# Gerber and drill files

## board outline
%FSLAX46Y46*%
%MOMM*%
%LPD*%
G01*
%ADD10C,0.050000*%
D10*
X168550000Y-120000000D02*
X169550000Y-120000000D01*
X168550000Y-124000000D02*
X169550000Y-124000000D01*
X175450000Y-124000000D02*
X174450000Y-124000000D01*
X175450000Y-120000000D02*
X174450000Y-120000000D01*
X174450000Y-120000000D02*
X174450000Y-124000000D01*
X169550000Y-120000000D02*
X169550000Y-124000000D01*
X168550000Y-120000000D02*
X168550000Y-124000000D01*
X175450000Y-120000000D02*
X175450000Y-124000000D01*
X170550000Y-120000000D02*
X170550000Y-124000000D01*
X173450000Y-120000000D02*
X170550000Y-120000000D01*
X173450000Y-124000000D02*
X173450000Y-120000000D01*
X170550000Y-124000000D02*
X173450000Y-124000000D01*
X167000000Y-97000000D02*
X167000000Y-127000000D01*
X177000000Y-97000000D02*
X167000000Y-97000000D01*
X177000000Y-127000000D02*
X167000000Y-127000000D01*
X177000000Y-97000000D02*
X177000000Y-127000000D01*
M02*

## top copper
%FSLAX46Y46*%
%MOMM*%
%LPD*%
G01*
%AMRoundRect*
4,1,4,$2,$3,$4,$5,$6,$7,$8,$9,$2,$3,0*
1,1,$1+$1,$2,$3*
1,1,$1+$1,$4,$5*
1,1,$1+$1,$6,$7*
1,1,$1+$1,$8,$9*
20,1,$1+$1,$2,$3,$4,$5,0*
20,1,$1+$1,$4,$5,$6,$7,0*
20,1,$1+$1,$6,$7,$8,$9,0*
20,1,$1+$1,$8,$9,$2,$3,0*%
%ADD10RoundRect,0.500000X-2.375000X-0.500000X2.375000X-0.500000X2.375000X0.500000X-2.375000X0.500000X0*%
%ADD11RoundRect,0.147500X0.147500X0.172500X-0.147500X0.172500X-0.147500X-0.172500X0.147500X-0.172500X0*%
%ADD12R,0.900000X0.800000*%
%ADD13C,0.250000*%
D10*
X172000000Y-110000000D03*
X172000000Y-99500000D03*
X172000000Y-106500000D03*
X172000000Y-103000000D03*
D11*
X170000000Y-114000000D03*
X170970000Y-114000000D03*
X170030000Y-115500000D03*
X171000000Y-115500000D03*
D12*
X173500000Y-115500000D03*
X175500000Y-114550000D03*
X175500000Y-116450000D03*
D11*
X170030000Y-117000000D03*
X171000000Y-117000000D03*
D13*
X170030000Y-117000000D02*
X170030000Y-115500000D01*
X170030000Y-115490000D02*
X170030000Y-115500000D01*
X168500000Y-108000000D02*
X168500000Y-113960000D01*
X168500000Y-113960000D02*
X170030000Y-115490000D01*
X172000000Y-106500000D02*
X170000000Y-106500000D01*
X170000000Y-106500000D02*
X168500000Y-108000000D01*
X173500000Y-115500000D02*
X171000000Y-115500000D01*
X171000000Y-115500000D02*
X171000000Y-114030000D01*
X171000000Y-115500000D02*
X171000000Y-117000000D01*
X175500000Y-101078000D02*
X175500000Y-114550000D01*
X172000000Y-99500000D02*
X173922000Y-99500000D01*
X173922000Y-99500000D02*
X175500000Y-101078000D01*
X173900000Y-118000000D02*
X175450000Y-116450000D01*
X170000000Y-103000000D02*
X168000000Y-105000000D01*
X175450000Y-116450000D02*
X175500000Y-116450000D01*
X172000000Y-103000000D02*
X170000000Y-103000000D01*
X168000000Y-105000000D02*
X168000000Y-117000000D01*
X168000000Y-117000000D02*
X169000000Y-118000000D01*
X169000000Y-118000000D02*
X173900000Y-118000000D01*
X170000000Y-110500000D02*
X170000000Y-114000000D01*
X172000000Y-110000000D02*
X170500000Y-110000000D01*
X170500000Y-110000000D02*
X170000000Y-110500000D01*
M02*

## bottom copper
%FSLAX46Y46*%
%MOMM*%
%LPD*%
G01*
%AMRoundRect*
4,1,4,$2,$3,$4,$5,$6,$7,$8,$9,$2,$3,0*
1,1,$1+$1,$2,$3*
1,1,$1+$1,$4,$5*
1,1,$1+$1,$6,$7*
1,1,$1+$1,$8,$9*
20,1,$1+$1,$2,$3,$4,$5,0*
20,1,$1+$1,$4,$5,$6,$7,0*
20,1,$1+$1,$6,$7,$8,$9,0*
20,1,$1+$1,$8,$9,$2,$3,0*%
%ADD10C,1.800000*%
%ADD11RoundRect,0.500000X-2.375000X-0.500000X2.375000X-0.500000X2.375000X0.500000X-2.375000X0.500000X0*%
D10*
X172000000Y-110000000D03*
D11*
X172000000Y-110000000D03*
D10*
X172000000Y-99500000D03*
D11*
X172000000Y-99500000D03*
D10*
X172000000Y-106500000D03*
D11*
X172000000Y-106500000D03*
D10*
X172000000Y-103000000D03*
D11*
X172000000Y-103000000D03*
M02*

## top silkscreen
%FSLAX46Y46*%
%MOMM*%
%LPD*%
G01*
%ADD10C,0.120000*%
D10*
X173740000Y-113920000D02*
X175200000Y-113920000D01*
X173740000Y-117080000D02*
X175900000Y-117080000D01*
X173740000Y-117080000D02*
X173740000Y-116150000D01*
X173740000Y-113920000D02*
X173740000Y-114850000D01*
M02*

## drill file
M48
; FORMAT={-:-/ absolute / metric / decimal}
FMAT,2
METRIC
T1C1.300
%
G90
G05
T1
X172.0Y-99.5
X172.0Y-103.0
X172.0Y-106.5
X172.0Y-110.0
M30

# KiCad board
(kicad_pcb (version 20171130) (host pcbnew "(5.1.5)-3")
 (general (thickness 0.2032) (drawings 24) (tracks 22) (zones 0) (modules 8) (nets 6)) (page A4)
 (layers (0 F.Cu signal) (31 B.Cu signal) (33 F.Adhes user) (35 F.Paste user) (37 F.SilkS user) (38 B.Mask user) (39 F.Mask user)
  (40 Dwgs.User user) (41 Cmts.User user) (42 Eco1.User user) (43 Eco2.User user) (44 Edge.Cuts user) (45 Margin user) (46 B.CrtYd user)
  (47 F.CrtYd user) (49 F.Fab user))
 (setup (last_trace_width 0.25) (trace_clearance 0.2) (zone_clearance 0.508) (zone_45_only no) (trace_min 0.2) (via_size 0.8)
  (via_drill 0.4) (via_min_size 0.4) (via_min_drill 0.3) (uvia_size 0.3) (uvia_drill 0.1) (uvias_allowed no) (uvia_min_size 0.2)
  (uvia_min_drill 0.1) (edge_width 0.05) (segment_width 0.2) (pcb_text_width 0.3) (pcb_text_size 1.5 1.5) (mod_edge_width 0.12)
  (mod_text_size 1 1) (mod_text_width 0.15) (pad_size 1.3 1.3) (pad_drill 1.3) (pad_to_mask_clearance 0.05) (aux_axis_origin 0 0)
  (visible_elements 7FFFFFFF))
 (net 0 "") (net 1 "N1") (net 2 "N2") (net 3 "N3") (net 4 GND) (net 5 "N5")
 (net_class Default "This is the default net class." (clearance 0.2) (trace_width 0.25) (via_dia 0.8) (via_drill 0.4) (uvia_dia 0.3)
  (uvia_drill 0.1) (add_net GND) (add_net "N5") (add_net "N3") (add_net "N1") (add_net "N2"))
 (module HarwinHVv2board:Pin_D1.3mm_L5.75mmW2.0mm (layer F.Cu) (at 172 110)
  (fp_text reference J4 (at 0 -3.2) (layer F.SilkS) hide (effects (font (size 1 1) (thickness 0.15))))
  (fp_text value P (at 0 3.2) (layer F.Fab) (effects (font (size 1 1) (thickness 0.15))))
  (pad 2 smd circle (at 0 0) (size 1.8 1.8) (layers B.Cu F.Paste F.Mask))
  (pad 1 thru_hole roundrect (at 0 0) (size 5.75 2) (drill 1.3) (layers F.Cu F.Mask) (roundrect_rratio 0.25) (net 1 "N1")))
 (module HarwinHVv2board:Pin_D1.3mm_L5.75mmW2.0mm (layer F.Cu) (at 172 99.5)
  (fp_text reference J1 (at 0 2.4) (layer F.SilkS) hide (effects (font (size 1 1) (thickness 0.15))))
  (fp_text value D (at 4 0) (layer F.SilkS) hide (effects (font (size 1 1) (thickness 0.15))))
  (pad 2 smd circle (at 0 0) (size 1.8 1.8) (layers B.Cu F.Paste F.Mask))
  (pad 1 thru_hole roundrect (at 0 0) (size 5.75 2) (drill 1.3) (layers F.Cu F.Mask) (roundrect_rratio 0.25) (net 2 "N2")))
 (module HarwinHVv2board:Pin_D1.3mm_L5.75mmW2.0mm (layer F.Cu) (at 172 106.5)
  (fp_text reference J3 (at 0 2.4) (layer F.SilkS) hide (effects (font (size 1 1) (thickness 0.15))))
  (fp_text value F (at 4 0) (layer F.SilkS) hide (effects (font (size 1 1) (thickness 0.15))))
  (pad 2 smd circle (at 0 0) (size 1.8 1.8) (layers B.Cu F.Paste F.Mask) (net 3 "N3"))
  (pad 1 thru_hole roundrect (at 0 0) (size 5.75 2) (drill 1.3) (layers F.Cu F.Mask) (roundrect_rratio 0.25) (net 3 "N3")))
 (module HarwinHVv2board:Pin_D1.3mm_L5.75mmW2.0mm (layer F.Cu) (at 172 103)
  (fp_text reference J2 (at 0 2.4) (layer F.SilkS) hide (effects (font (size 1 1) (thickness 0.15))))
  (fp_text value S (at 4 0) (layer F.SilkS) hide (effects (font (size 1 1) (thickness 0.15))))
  (pad 2 smd circle (at 0 0) (size 1.8 1.8) (layers B.Cu F.Paste F.Mask))
  (pad 1 thru_hole roundrect (at 0 0) (size 5.75 2) (drill 1.3) (layers F.Cu F.Mask) (roundrect_rratio 0.25) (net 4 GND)))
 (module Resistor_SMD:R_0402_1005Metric (layer F.Cu) (at 170.485 114 180)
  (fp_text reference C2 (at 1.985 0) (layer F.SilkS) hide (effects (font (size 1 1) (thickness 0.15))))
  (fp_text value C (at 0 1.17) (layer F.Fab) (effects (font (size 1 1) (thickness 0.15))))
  (pad 2 smd roundrect (at 0.485 0 180) (size 0.59 0.64) (layers F.Cu F.Paste F.Mask) (roundrect_rratio 0.25) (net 1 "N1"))
  (pad 1 smd roundrect (at -0.485 0 180) (size 0.59 0.64) (layers F.Cu F.Paste F.Mask) (roundrect_rratio 0.25) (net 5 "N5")))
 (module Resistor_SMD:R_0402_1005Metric (layer F.Cu) (at 170.515 115.5 180)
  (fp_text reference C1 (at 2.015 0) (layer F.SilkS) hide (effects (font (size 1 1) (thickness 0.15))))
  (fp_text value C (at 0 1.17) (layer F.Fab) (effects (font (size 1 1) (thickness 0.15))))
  (pad 2 smd roundrect (at 0.485 0 180) (size 0.59 0.64) (layers F.Cu F.Paste F.Mask) (roundrect_rratio 0.25) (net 3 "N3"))
  (pad 1 smd roundrect (at -0.485 0 180) (size 0.59 0.64) (layers F.Cu F.Paste F.Mask) (roundrect_rratio 0.25) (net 5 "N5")))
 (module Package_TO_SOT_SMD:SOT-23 (layer F.Cu) (at 174.5 115.5 180)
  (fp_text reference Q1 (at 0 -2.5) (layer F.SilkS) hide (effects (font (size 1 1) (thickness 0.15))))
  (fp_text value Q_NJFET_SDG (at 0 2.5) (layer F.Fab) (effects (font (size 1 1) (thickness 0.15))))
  (fp_line (start 0.76 1.58) (end -0.7 1.58) (layer F.SilkS) (width 0.12))
  (fp_line (start 0.76 -1.58) (end -1.4 -1.58) (layer F.SilkS) (width 0.12))
  (fp_line (start 0.76 -1.58) (end 0.76 -0.65) (layer F.SilkS) (width 0.12))
  (fp_line (start 0.76 1.58) (end 0.76 0.65) (layer F.SilkS) (width 0.12))
  (pad 3 smd rect (at 1 0 180) (size 0.9 0.8) (layers F.Cu F.Paste F.Mask) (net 5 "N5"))
  (pad 2 smd rect (at -1 0.95 180) (size 0.9 0.8) (layers F.Cu F.Paste F.Mask) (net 2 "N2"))
  (pad 1 smd rect (at -1 -0.95 180) (size 0.9 0.8) (layers F.Cu F.Paste F.Mask) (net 4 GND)))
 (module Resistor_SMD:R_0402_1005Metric (layer F.Cu) (at 170.515 117 180)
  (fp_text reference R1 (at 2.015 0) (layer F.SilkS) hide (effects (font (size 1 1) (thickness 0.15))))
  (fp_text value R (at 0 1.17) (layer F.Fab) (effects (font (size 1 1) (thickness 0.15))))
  (pad 2 smd roundrect (at 0.485 0 180) (size 0.59 0.64) (layers F.Cu F.Paste F.Mask) (roundrect_rratio 0.25) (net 3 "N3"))
  (pad 1 smd roundrect (at -0.485 0 180) (size 0.59 0.64) (layers F.Cu F.Paste F.Mask) (roundrect_rratio 0.25) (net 5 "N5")))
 (gr_line (start 168.55 120) (end 169.55 120) (layer Edge.Cuts) (width 0.05))
 (gr_line (start 168.55 124) (end 169.55 124) (layer Edge.Cuts) (width 0.05))
 (gr_line (start 175.45 124) (end 174.45 124) (layer Edge.Cuts) (width 0.05))
 (gr_line (start 175.45 120) (end 174.45 120) (layer Edge.Cuts) (width 0.05))
 (gr_line (start 174.45 120) (end 174.45 124) (layer Edge.Cuts) (width 0.05))
 (gr_line (start 169.55 120) (end 169.55 124) (layer Edge.Cuts) (width 0.05))
 (gr_line (start 168.55 120) (end 168.55 124) (layer Edge.Cuts) (width 0.05))
 (gr_line (start 175.45 120) (end 175.45 124) (layer Edge.Cuts) (width 0.05))
 (gr_line (start 170.55 120) (end 170.55 124) (layer Edge.Cuts) (width 0.05))
 (gr_line (start 173.45 120) (end 170.55 120) (layer Edge.Cuts) (width 0.05))
 (gr_line (start 173.45 124) (end 173.45 120) (layer Edge.Cuts) (width 0.05))
 (gr_line (start 170.55 124) (end 173.45 124) (layer Edge.Cuts) (width 0.05))
 (gr_line (start 167 97) (end 167 127) (layer Edge.Cuts) (width 0.05))
 (gr_line (start 177 97) (end 167 97) (layer Edge.Cuts) (width 0.05))
 (gr_line (start 177 127) (end 167 127) (layer Edge.Cuts) (width 0.05))
 (gr_line (start 177 97) (end 177 127) (layer Edge.Cuts) (width 0.05))
 (segment (start 170.03 117) (end 170.03 115.5) (width 0.25) (layer F.Cu) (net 3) (status 30))
 (segment (start 170.03 115.49) (end 170.03 115.5) (width 0.25) (layer F.Cu) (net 3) (status 30))
 (segment (start 168.5 108) (end 168.5 113.96) (width 0.25) (layer F.Cu) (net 3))
 (segment (start 168.5 113.96) (end 170.03 115.49) (width 0.25) (layer F.Cu) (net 3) (status 20))
 (segment (start 172 106.5) (end 170 106.5) (width 0.25) (layer F.Cu) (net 3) (status 30))
 (segment (start 170 106.5) (end 168.5 108) (width 0.25) (layer F.Cu) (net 3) (status 10))
 (segment (start 173.5 115.5) (end 171 115.5) (width 0.25) (layer F.Cu) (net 5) (status 30))
 (segment (start 171 115.5) (end 171 114.03) (width 0.25) (layer F.Cu) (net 5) (status 30))
 (segment (start 171 115.5) (end 171 117) (width 0.25) (layer F.Cu) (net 5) (status 30))
 (segment (start 175.5 101.078) (end 175.5 114.55) (width 0.25) (layer F.Cu) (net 2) (status 20))
 (segment (start 172 99.5) (end 173.922 99.5) (width 0.25) (layer F.Cu) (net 2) (status 30))
 (segment (start 173.922 99.5) (end 175.5 101.078) (width 0.25) (layer F.Cu) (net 2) (status 10))
 (segment (start 173.9 118) (end 175.45 116.45) (width 0.25) (layer F.Cu) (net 4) (status 20))
 (segment (start 170 103) (end 168 105) (width 0.25) (layer F.Cu) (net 4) (status 10))
 (segment (start 175.45 116.45) (end 175.5 116.45) (width 0.25) (layer F.Cu) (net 4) (status 30))
 (segment (start 172 103) (end 170 103) (width 0.25) (layer F.Cu) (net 4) (status 30))
 (segment (start 168 105) (end 168 117) (width 0.25) (layer F.Cu) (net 4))
 (segment (start 168 117) (end 169 118) (width 0.25) (layer F.Cu) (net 4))
 (segment (start 169 118) (end 173.9 118) (width 0.25) (layer F.Cu) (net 4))
 (segment (start 170 110.5) (end 170 114) (width 0.25) (layer F.Cu) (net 1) (status 30))
 (segment (start 172 110) (end 170.5 110) (width 0.25) (layer F.Cu) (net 1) (status 30))
 (segment (start 170.5 110) (end 170 110.5) (width 0.25) (layer F.Cu) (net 1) (status 30)))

